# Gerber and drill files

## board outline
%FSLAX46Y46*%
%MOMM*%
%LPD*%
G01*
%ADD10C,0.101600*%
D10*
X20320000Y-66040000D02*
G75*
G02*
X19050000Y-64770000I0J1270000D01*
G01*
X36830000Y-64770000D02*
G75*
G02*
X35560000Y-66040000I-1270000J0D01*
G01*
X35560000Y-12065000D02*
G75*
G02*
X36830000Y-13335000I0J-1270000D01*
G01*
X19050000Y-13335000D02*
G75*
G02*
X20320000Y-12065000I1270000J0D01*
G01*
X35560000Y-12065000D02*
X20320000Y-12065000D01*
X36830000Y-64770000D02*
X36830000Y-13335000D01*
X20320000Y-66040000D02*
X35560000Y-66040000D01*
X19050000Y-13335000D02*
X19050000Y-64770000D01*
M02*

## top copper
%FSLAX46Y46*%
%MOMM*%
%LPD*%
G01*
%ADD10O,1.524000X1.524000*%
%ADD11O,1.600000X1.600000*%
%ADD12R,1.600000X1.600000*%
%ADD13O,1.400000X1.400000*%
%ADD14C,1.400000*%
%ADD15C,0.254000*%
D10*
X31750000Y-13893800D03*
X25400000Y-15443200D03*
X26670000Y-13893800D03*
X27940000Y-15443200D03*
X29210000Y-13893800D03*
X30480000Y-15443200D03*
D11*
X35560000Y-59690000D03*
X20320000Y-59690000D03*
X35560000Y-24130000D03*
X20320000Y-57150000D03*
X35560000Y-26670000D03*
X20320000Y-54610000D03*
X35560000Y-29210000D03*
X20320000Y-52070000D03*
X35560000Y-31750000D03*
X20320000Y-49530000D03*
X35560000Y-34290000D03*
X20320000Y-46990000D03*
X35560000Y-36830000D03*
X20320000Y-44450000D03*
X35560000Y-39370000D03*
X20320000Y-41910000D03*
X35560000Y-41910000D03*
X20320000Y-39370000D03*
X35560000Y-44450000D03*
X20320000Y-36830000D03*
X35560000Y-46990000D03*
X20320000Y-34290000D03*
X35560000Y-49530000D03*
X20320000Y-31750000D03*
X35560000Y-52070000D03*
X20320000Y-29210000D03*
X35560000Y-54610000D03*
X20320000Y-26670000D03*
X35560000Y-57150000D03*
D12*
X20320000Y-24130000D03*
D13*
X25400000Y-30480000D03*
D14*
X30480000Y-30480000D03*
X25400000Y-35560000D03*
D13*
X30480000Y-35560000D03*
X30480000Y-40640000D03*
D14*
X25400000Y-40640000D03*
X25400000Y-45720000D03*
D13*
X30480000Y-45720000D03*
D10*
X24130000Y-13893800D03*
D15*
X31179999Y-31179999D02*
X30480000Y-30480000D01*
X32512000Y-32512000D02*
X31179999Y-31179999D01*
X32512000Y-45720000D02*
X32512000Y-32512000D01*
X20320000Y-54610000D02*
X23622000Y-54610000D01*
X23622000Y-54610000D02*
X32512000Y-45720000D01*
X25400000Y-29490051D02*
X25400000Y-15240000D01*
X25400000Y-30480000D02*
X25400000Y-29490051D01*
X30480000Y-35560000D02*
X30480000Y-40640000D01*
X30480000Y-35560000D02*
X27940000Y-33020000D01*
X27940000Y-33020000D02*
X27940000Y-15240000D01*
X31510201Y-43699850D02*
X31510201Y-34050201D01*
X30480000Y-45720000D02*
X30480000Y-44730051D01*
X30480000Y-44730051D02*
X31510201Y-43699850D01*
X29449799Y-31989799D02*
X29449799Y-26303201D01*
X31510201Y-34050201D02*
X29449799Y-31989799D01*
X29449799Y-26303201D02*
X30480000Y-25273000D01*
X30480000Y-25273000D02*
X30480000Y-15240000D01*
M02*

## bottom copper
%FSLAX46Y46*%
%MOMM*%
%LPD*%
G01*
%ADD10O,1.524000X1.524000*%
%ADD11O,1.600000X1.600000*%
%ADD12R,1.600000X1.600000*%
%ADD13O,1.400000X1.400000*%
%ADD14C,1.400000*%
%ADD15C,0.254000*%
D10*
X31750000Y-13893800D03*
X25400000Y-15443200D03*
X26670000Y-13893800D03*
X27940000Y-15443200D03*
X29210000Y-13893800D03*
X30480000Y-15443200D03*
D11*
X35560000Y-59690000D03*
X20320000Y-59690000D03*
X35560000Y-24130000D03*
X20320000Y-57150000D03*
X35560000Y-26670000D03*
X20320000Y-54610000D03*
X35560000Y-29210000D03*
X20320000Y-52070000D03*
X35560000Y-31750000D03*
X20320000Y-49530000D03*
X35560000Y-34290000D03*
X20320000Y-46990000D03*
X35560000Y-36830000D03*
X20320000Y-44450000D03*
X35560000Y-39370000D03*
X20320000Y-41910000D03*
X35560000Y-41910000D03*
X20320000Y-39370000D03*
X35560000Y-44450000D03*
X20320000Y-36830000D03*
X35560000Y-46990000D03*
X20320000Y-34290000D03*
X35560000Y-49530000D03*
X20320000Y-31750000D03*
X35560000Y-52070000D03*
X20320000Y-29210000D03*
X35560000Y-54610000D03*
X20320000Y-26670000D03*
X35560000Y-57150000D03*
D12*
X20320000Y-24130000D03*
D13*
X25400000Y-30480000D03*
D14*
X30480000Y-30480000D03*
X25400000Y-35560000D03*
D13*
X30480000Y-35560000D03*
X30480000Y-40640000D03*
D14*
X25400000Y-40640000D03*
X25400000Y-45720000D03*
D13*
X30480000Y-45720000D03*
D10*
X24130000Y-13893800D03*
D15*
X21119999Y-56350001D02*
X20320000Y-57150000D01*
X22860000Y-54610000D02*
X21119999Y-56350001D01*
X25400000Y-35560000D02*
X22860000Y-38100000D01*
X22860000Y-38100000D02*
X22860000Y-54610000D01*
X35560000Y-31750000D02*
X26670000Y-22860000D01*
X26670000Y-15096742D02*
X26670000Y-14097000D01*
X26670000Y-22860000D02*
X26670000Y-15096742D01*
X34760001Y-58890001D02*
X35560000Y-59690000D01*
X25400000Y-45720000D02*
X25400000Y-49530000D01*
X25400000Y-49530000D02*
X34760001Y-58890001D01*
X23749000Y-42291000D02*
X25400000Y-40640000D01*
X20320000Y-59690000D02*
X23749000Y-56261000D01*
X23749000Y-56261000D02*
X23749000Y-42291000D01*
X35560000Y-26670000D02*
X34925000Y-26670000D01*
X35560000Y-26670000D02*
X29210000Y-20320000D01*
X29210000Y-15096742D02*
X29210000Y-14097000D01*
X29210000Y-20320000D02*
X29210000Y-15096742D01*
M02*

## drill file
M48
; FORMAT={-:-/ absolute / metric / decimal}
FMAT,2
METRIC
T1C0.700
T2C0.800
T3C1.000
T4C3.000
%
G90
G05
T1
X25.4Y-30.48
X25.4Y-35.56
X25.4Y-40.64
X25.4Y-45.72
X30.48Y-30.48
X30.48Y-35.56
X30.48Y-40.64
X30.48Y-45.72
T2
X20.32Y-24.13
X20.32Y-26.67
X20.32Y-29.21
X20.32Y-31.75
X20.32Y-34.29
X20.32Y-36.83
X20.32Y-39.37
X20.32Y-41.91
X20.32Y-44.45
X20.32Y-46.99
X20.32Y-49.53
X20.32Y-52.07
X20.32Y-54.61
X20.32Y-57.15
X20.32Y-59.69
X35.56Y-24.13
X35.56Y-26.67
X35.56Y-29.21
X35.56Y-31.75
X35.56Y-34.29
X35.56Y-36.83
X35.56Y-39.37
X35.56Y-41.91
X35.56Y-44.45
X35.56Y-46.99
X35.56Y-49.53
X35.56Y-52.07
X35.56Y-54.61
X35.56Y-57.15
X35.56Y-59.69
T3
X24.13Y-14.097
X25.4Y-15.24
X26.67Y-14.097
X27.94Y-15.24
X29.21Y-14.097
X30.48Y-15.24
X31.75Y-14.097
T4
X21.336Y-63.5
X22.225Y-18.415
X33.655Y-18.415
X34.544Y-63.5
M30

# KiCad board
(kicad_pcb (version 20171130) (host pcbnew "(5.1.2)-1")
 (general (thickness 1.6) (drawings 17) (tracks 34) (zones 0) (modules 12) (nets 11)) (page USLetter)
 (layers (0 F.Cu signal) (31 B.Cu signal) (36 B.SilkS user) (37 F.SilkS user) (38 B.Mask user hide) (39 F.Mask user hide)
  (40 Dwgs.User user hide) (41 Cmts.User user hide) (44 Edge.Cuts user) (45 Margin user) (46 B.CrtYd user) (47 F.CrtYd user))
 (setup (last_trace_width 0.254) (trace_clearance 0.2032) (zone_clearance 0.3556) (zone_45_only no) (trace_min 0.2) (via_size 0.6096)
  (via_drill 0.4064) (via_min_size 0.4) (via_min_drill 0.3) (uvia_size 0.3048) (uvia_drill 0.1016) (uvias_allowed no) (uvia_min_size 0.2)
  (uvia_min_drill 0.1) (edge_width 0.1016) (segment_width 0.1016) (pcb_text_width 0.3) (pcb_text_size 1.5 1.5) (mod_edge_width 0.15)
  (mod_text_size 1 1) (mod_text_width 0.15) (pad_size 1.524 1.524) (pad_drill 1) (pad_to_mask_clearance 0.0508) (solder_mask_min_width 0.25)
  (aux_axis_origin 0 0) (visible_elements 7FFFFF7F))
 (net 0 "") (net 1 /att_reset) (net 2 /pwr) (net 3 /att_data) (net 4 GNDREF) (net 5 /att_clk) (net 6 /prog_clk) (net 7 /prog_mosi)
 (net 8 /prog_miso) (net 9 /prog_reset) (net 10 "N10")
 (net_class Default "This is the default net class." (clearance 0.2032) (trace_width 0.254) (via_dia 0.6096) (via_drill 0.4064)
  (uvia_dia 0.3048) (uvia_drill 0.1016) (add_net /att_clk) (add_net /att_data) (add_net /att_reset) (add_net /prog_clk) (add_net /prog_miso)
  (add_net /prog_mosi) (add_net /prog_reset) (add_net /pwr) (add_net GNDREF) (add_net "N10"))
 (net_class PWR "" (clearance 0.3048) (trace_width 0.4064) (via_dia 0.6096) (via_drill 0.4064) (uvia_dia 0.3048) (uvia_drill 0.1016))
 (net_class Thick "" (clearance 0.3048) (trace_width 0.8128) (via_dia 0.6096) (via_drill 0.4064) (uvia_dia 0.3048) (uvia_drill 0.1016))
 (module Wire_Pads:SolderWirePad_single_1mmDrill (layer F.Cu) (at 31.75 14.097 90)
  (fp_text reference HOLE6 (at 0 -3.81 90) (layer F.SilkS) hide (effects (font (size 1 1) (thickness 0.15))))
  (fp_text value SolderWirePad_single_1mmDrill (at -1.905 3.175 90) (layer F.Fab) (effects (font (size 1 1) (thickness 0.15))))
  (pad 1 thru_hole oval (at 0 0 90) (size 1.524 1.524) (drill 1 (offset 0.2032 0)) (layers *.Cu *.Mask)))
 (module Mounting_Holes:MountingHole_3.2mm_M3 (layer F.Cu) (at 33.655 18.415)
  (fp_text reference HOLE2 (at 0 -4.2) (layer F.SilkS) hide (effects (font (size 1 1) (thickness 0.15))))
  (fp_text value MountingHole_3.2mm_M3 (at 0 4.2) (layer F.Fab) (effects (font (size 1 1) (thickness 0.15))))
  (pad "" np_thru_hole circle (at 0 0) (size 3 3) (drill 3) (layers *.Cu *.Mask)))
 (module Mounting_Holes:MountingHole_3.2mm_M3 (layer F.Cu) (at 34.544 63.5)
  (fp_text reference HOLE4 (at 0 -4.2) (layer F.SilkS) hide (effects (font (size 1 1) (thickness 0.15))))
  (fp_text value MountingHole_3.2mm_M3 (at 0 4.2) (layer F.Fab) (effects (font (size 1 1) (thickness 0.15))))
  (pad "" np_thru_hole circle (at 0 0) (size 3 3) (drill 3) (layers *.Cu *.Mask)))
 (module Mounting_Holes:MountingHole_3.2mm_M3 (layer F.Cu) (at 21.336 63.5)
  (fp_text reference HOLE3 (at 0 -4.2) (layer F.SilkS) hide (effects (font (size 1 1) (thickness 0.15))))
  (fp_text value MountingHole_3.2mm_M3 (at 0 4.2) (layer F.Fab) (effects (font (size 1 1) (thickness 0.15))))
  (pad "" np_thru_hole circle (at 0 0) (size 3 3) (drill 3) (layers *.Cu *.Mask)))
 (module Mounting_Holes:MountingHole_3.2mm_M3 (layer F.Cu) (at 22.225 18.415)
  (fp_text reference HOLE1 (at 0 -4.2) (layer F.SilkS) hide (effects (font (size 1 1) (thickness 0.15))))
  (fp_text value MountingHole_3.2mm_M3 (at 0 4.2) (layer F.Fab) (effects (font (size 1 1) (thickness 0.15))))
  (pad "" np_thru_hole circle (at 0 0) (size 3 3) (drill 3) (layers *.Cu *.Mask)))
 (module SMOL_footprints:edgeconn (layer F.Cu) (at 25.4 14.605 90)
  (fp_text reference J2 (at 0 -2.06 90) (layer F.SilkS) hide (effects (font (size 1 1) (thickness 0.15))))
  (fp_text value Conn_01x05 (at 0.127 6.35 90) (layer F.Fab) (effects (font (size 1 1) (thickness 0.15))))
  (pad 1 thru_hole oval (at -0.635 0 90) (size 1.524 1.524) (drill 1 (offset -0.2032 0)) (layers *.Cu *.Mask) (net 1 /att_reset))
  (pad 2 thru_hole oval (at 0.508 1.27 90) (size 1.524 1.524) (drill 1 (offset 0.2032 0)) (layers *.Cu *.Mask) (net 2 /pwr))
  (pad 3 thru_hole oval (at -0.635 2.54 90) (size 1.524 1.524) (drill 1 (offset -0.2032 0)) (layers *.Cu *.Mask) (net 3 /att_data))
  (pad 4 thru_hole oval (at 0.508 3.81 90) (size 1.524 1.524) (drill 1 (offset 0.2032 0)) (layers *.Cu *.Mask) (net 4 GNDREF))
  (pad 5 thru_hole oval (at -0.635 5.08 90) (size 1.524 1.524) (drill 1 (offset -0.2032 0)) (layers *.Cu *.Mask) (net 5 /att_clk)))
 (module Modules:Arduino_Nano (layer F.Cu) (at 20.32 24.13)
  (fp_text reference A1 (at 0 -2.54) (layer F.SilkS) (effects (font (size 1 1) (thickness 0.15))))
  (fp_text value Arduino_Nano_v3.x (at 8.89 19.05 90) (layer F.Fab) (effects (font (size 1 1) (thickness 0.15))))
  (pad 16 thru_hole oval (at 15.24 35.56) (size 1.6 1.6) (drill 0.8) (layers *.Cu *.Mask) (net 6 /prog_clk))
  (pad 15 thru_hole oval (at 0 35.56) (size 1.6 1.6) (drill 0.8) (layers *.Cu *.Mask) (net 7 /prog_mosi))
  (pad 30 thru_hole oval (at 15.24 0) (size 1.6 1.6) (drill 0.8) (layers *.Cu *.Mask))
  (pad 14 thru_hole oval (at 0 33.02) (size 1.6 1.6) (drill 0.8) (layers *.Cu *.Mask) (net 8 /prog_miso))
  (pad 29 thru_hole oval (at 15.24 2.54) (size 1.6 1.6) (drill 0.8) (layers *.Cu *.Mask) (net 4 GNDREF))
  (pad 13 thru_hole oval (at 0 30.48) (size 1.6 1.6) (drill 0.8) (layers *.Cu *.Mask) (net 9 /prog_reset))
  (pad 28 thru_hole oval (at 15.24 5.08) (size 1.6 1.6) (drill 0.8) (layers *.Cu *.Mask))
  (pad 12 thru_hole oval (at 0 27.94) (size 1.6 1.6) (drill 0.8) (layers *.Cu *.Mask))
  (pad 27 thru_hole oval (at 15.24 7.62) (size 1.6 1.6) (drill 0.8) (layers *.Cu *.Mask) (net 2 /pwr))
  (pad 11 thru_hole oval (at 0 25.4) (size 1.6 1.6) (drill 0.8) (layers *.Cu *.Mask))
  (pad 26 thru_hole oval (at 15.24 10.16) (size 1.6 1.6) (drill 0.8) (layers *.Cu *.Mask))
  (pad 10 thru_hole oval (at 0 22.86) (size 1.6 1.6) (drill 0.8) (layers *.Cu *.Mask))
  (pad 25 thru_hole oval (at 15.24 12.7) (size 1.6 1.6) (drill 0.8) (layers *.Cu *.Mask))
  (pad 9 thru_hole oval (at 0 20.32) (size 1.6 1.6) (drill 0.8) (layers *.Cu *.Mask))
  (pad 24 thru_hole oval (at 15.24 15.24) (size 1.6 1.6) (drill 0.8) (layers *.Cu *.Mask))
  (pad 8 thru_hole oval (at 0 17.78) (size 1.6 1.6) (drill 0.8) (layers *.Cu *.Mask))
  (pad 23 thru_hole oval (at 15.24 17.78) (size 1.6 1.6) (drill 0.8) (layers *.Cu *.Mask))
  (pad 7 thru_hole oval (at 0 15.24) (size 1.6 1.6) (drill 0.8) (layers *.Cu *.Mask))
  (pad 22 thru_hole oval (at 15.24 20.32) (size 1.6 1.6) (drill 0.8) (layers *.Cu *.Mask))
  (pad 6 thru_hole oval (at 0 12.7) (size 1.6 1.6) (drill 0.8) (layers *.Cu *.Mask))
  (pad 21 thru_hole oval (at 15.24 22.86) (size 1.6 1.6) (drill 0.8) (layers *.Cu *.Mask))
  (pad 5 thru_hole oval (at 0 10.16) (size 1.6 1.6) (drill 0.8) (layers *.Cu *.Mask))
  (pad 20 thru_hole oval (at 15.24 25.4) (size 1.6 1.6) (drill 0.8) (layers *.Cu *.Mask))
  (pad 4 thru_hole oval (at 0 7.62) (size 1.6 1.6) (drill 0.8) (layers *.Cu *.Mask) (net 4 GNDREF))
  (pad 19 thru_hole oval (at 15.24 27.94) (size 1.6 1.6) (drill 0.8) (layers *.Cu *.Mask))
  (pad 3 thru_hole oval (at 0 5.08) (size 1.6 1.6) (drill 0.8) (layers *.Cu *.Mask))
  (pad 18 thru_hole oval (at 15.24 30.48) (size 1.6 1.6) (drill 0.8) (layers *.Cu *.Mask))
  (pad 2 thru_hole oval (at 0 2.54) (size 1.6 1.6) (drill 0.8) (layers *.Cu *.Mask))
  (pad 17 thru_hole oval (at 15.24 33.02) (size 1.6 1.6) (drill 0.8) (layers *.Cu *.Mask) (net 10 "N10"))
  (pad 1 thru_hole rect (at 0 0) (size 1.6 1.6) (drill 0.8) (layers *.Cu *.Mask)))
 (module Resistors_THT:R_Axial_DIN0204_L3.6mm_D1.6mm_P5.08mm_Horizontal (layer F.Cu) (at 30.48 30.48 180)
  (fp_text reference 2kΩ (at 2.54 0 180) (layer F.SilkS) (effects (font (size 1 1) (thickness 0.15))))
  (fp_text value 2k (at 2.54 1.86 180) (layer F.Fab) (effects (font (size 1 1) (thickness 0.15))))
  (pad 2 thru_hole oval (at 5.08 0 180) (size 1.4 1.4) (drill 0.7) (layers *.Cu *.Mask) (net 1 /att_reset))
  (pad 1 thru_hole circle (at 0 0 180) (size 1.4 1.4) (drill 0.7) (layers *.Cu *.Mask) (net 9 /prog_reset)))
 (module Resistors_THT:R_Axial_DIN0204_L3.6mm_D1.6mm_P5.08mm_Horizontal (layer F.Cu) (at 25.4 35.56)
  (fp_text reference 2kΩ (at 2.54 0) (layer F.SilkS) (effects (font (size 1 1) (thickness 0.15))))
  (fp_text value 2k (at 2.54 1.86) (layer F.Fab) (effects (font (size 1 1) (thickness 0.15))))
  (pad 1 thru_hole circle (at 0 0) (size 1.4 1.4) (drill 0.7) (layers *.Cu *.Mask) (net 8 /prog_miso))
  (pad 2 thru_hole oval (at 5.08 0) (size 1.4 1.4) (drill 0.7) (layers *.Cu *.Mask) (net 3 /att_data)))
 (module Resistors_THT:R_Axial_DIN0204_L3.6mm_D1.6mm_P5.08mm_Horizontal (layer F.Cu) (at 25.4 40.64)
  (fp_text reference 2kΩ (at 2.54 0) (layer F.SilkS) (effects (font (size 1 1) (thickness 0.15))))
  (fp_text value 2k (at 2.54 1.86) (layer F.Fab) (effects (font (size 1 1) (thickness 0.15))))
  (pad 2 thru_hole oval (at 5.08 0) (size 1.4 1.4) (drill 0.7) (layers *.Cu *.Mask) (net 3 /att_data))
  (pad 1 thru_hole circle (at 0 0) (size 1.4 1.4) (drill 0.7) (layers *.Cu *.Mask) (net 7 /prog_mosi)))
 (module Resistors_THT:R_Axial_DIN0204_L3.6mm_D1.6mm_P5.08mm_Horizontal (layer F.Cu) (at 25.4 45.72)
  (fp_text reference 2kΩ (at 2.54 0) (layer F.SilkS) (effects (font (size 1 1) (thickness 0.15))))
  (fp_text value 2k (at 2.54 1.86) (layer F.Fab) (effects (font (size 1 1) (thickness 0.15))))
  (pad 1 thru_hole circle (at 0 0) (size 1.4 1.4) (drill 0.7) (layers *.Cu *.Mask) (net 6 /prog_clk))
  (pad 2 thru_hole oval (at 5.08 0) (size 1.4 1.4) (drill 0.7) (layers *.Cu *.Mask) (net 5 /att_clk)))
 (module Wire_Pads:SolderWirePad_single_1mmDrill (layer F.Cu) (at 24.13 14.097 90)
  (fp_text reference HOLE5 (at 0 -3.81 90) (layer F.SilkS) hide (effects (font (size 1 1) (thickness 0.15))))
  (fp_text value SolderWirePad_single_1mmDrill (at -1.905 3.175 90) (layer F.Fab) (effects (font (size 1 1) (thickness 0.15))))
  (pad 1 thru_hole oval (at 0 0 90) (size 1.524 1.524) (drill 1 (offset 0.2032 0)) (layers *.Cu *.Mask)))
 (gr_arc (start 20.32 64.77) (end 19.05 64.77) (angle -90) (layer Edge.Cuts) (width 0.1016))
 (gr_arc (start 35.56 64.77) (end 35.56 66.04) (angle -90) (layer Edge.Cuts) (width 0.1016))
 (gr_arc (start 35.56 13.335) (end 36.83 13.335) (angle -90) (layer Edge.Cuts) (width 0.1016))
 (gr_arc (start 20.32 13.335) (end 20.32 12.065) (angle -90) (layer Edge.Cuts) (width 0.1016))
 (gr_line (start 35.56 12.065) (end 20.32 12.065) (layer Edge.Cuts) (width 0.1016))
 (gr_line (start 36.83 64.77) (end 36.83 13.335) (layer Edge.Cuts) (width 0.1016))
 (gr_line (start 20.32 66.04) (end 35.56 66.04) (layer Edge.Cuts) (width 0.1016))
 (gr_line (start 19.05 13.335) (end 19.05 64.77) (layer Edge.Cuts) (width 0.1016))
 (segment (start 21.119999 56.350001) (end 20.32 57.15) (width 0.254) (layer B.Cu) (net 8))
 (segment (start 22.86 54.61) (end 21.119999 56.350001) (width 0.254) (layer B.Cu) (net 8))
 (segment (start 25.4 35.56) (end 22.86 38.1) (width 0.254) (layer B.Cu) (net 8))
 (segment (start 22.86 38.1) (end 22.86 54.61) (width 0.254) (layer B.Cu) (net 8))
 (segment (start 35.56 31.75) (end 26.67 22.86) (width 0.254) (layer B.Cu) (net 2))
 (segment (start 26.67 15.096742) (end 26.67 14.097) (width 0.254) (layer B.Cu) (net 2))
 (segment (start 26.67 22.86) (end 26.67 15.096742) (width 0.254) (layer B.Cu) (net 2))
 (segment (start 34.760001 58.890001) (end 35.56 59.69) (width 0.254) (layer B.Cu) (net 6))
 (segment (start 25.4 45.72) (end 25.4 49.53) (width 0.254) (layer B.Cu) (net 6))
 (segment (start 25.4 49.53) (end 34.760001 58.890001) (width 0.254) (layer B.Cu) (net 6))
 (segment (start 23.749 42.291) (end 25.4 40.64) (width 0.254) (layer B.Cu) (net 7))
 (segment (start 20.32 59.69) (end 23.749 56.261) (width 0.254) (layer B.Cu) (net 7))
 (segment (start 23.749 56.261) (end 23.749 42.291) (width 0.254) (layer B.Cu) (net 7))
 (segment (start 31.179999 31.179999) (end 30.48 30.48) (width 0.254) (layer F.Cu) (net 9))
 (segment (start 32.512 32.512) (end 31.179999 31.179999) (width 0.254) (layer F.Cu) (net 9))
 (segment (start 32.512 45.72) (end 32.512 32.512) (width 0.254) (layer F.Cu) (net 9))
 (segment (start 20.32 54.61) (end 23.622 54.61) (width 0.254) (layer F.Cu) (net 9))
 (segment (start 23.622 54.61) (end 32.512 45.72) (width 0.254) (layer F.Cu) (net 9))
 (segment (start 25.4 29.490051) (end 25.4 15.24) (width 0.254) (layer F.Cu) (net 1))
 (segment (start 25.4 30.48) (end 25.4 29.490051) (width 0.254) (layer F.Cu) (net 1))
 (segment (start 30.48 35.56) (end 30.48 40.64) (width 0.254) (layer F.Cu) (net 3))
 (segment (start 30.48 35.56) (end 27.94 33.02) (width 0.254) (layer F.Cu) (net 3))
 (segment (start 27.94 33.02) (end 27.94 15.24) (width 0.254) (layer F.Cu) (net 3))
 (segment (start 35.56 26.67) (end 34.925 26.67) (width 0.254) (layer B.Cu) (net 4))
 (segment (start 35.56 26.67) (end 29.21 20.32) (width 0.254) (layer B.Cu) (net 4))
 (segment (start 29.21 15.096742) (end 29.21 14.097) (width 0.254) (layer B.Cu) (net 4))
 (segment (start 29.21 20.32) (end 29.21 15.096742) (width 0.254) (layer B.Cu) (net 4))
 (segment (start 31.510201 43.69985) (end 31.510201 34.050201) (width 0.254) (layer F.Cu) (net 5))
 (segment (start 30.48 45.72) (end 30.48 44.730051) (width 0.254) (layer F.Cu) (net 5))
 (segment (start 30.48 44.730051) (end 31.510201 43.69985) (width 0.254) (layer F.Cu) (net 5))
 (segment (start 29.449799 31.989799) (end 29.449799 26.303201) (width 0.254) (layer F.Cu) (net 5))
 (segment (start 31.510201 34.050201) (end 29.449799 31.989799) (width 0.254) (layer F.Cu) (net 5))
 (segment (start 29.449799 26.303201) (end 30.48 25.273) (width 0.254) (layer F.Cu) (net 5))
 (segment (start 30.48 25.273) (end 30.48 15.24) (width 0.254) (layer F.Cu) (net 5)))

